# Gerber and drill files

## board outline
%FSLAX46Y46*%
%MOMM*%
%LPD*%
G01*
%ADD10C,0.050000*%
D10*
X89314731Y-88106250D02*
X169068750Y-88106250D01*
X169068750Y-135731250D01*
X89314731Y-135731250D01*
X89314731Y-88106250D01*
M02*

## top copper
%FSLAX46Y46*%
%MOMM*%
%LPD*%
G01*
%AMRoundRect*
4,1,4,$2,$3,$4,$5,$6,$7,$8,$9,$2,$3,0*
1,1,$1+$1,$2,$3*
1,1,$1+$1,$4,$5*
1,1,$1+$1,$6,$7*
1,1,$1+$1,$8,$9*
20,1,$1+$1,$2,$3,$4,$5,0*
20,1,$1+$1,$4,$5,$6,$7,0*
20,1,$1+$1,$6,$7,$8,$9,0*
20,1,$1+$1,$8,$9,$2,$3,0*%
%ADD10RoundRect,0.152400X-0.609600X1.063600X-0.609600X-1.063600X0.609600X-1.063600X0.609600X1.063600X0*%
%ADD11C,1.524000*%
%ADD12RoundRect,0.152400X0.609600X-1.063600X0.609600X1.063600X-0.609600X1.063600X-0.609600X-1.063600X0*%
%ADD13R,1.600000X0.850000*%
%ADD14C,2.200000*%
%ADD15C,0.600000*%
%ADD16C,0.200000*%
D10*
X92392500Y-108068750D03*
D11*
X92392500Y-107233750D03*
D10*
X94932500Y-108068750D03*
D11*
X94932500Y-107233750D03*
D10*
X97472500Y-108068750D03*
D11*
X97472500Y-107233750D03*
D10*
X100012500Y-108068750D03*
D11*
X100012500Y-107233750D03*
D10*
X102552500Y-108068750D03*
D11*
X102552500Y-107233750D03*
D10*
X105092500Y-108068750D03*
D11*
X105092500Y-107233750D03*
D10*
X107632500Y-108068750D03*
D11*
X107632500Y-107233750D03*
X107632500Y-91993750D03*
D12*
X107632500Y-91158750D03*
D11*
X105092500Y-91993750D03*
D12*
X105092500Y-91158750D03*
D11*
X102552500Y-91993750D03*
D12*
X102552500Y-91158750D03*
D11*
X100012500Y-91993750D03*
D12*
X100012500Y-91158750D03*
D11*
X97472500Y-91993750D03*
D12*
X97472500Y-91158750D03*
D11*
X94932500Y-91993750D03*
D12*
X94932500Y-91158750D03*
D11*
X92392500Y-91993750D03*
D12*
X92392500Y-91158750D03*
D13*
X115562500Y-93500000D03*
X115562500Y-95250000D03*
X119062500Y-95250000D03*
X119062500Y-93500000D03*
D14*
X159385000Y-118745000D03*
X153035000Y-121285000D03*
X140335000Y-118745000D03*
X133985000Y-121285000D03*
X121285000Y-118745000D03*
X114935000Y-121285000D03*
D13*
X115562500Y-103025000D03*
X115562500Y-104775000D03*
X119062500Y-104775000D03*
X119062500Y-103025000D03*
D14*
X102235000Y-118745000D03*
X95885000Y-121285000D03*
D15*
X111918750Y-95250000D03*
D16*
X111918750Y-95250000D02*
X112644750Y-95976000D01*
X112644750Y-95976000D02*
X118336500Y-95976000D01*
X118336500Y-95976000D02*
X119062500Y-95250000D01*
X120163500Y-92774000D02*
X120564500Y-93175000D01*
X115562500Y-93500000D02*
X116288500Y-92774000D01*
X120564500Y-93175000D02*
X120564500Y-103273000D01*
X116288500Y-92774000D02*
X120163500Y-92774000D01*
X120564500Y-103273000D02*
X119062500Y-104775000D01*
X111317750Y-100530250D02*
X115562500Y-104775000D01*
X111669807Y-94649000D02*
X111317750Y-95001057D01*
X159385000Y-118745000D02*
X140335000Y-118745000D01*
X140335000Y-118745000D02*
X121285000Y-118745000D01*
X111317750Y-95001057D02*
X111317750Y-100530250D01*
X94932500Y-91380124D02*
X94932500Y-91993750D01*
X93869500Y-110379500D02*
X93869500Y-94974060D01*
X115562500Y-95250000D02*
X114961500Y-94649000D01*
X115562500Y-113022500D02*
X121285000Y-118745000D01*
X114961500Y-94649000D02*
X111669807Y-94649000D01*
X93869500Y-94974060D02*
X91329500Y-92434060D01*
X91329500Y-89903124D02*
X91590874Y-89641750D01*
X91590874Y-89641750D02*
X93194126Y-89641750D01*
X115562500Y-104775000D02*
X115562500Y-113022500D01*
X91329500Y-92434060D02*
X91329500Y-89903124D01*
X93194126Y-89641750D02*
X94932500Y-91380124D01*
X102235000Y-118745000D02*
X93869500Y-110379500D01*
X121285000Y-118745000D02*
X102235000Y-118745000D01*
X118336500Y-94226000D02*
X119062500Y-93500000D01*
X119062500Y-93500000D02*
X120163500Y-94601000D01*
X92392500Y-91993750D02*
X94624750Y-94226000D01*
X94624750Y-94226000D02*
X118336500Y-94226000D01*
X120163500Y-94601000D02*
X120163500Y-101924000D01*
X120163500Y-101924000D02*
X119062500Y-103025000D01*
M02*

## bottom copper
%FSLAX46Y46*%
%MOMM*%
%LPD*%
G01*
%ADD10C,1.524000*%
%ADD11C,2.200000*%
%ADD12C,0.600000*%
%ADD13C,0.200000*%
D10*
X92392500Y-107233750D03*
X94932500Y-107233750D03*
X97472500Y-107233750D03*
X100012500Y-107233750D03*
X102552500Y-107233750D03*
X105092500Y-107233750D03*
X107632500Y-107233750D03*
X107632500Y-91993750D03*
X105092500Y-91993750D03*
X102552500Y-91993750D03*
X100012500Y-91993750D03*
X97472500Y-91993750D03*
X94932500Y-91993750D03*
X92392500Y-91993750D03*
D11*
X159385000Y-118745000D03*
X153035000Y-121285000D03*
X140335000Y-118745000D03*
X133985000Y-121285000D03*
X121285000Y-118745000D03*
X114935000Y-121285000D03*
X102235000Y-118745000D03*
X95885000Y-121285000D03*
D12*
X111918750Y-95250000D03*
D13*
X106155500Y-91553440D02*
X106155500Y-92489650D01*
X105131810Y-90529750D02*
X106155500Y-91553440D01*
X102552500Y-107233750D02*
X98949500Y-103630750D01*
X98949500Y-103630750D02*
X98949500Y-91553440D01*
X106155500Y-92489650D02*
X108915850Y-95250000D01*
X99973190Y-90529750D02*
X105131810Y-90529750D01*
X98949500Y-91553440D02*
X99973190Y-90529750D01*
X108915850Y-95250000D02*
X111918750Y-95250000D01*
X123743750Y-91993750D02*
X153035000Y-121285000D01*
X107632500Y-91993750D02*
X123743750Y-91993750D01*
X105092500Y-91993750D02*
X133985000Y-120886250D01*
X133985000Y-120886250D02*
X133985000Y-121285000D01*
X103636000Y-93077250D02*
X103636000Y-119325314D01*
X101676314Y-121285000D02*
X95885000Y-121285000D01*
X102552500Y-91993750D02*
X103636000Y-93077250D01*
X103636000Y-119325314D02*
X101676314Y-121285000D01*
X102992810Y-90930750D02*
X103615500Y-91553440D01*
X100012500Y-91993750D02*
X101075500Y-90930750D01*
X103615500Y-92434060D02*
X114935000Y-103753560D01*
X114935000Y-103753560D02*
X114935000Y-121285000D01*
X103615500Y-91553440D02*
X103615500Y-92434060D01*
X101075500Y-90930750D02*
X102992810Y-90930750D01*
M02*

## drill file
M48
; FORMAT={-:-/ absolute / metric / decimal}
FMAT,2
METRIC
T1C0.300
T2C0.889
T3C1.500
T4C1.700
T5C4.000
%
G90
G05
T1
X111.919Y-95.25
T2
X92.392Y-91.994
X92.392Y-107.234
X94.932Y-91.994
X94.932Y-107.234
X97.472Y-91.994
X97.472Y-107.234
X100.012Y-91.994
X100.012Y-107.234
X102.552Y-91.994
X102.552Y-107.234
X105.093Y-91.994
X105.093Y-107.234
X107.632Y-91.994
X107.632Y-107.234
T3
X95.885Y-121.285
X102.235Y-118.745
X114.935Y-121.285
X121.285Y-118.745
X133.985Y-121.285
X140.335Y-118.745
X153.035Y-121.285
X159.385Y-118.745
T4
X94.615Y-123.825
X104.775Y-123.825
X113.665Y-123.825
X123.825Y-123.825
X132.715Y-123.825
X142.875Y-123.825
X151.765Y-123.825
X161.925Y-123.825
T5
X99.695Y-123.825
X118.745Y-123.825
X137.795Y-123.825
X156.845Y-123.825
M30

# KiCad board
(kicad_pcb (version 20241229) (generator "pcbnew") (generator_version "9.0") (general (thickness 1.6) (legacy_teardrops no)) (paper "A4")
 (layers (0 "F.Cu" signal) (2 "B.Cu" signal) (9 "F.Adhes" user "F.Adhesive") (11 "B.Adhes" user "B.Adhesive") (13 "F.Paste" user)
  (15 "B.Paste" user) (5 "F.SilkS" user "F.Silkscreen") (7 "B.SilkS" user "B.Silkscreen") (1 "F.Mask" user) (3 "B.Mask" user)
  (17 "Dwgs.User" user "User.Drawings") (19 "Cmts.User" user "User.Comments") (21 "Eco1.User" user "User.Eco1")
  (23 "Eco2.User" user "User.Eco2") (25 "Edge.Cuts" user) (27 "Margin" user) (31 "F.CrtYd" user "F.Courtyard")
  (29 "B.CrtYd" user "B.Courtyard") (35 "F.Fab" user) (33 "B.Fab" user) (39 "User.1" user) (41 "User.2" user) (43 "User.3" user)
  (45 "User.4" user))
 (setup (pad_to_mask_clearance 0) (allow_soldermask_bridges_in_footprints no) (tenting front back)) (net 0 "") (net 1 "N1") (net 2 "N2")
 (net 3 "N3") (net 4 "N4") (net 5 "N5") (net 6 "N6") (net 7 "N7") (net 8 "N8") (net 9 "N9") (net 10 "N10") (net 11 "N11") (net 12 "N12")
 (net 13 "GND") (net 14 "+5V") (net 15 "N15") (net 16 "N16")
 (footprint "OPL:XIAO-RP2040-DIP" (layer "F.Cu") (at 100.0125 99.61375 90)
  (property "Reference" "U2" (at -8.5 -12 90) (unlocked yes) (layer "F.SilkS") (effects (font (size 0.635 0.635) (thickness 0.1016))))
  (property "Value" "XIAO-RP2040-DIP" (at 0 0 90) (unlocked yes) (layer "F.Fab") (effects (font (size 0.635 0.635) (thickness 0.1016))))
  (pad "1" smd roundrect (at -8.455 -7.62 270) (size 2.432 1.524) (layers "F.Cu" "F.Mask") (roundrect_rratio 0.1) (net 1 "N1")
   (thermal_bridge_angle 45))
  (pad "1" thru_hole circle (at -7.62 -7.62 270) (size 1.524 1.524) (drill 0.889) (layers "*.Cu" "*.Mask") (remove_unused_layers no)
   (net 1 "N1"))
  (pad "2" smd roundrect (at -8.455 -5.08 270) (size 2.432 1.524) (layers "F.Cu" "F.Mask") (roundrect_rratio 0.1) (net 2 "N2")
   (thermal_bridge_angle 45))
  (pad "2" thru_hole circle (at -7.62 -5.08 270) (size 1.524 1.524) (drill 0.889) (layers "*.Cu" "*.Mask") (remove_unused_layers no)
   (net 2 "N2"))
  (pad "3" smd roundrect (at -8.455 -2.54 270) (size 2.432 1.524) (layers "F.Cu" "F.Mask") (roundrect_rratio 0.1) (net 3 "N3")
   (thermal_bridge_angle 45))
  (pad "3" thru_hole circle (at -7.62 -2.54 270) (size 1.524 1.524) (drill 0.889) (layers "*.Cu" "*.Mask") (remove_unused_layers no)
   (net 3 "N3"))
  (pad "4" smd roundrect (at -8.455 0 270) (size 2.432 1.524) (layers "F.Cu" "F.Mask") (roundrect_rratio 0.1) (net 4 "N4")
   (thermal_bridge_angle 45))
  (pad "4" thru_hole circle (at -7.62 0 270) (size 1.524 1.524) (drill 0.889) (layers "*.Cu" "*.Mask") (remove_unused_layers no)
   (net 4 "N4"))
  (pad "5" smd roundrect (at -8.455 2.54 270) (size 2.432 1.524) (layers "F.Cu" "F.Mask") (roundrect_rratio 0.1) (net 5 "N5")
   (thermal_bridge_angle 45))
  (pad "5" thru_hole circle (at -7.62 2.54 270) (size 1.524 1.524) (drill 0.889) (layers "*.Cu" "*.Mask") (remove_unused_layers no)
   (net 5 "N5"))
  (pad "6" smd roundrect (at -8.455 5.08 270) (size 2.432 1.524) (layers "F.Cu" "F.Mask") (roundrect_rratio 0.1) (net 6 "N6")
   (thermal_bridge_angle 45))
  (pad "6" thru_hole circle (at -7.62 5.08 270) (size 1.524 1.524) (drill 0.889) (layers "*.Cu" "*.Mask") (remove_unused_layers no)
   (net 6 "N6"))
  (pad "7" smd roundrect (at -8.455 7.62 270) (size 2.432 1.524) (layers "F.Cu" "F.Mask") (roundrect_rratio 0.1) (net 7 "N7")
   (thermal_bridge_angle 45))
  (pad "7" thru_hole circle (at -7.62 7.62 270) (size 1.524 1.524) (drill 0.889) (layers "*.Cu" "*.Mask") (remove_unused_layers no)
   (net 7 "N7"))
  (pad "8" thru_hole circle (at 7.62 7.62 90) (size 1.524 1.524) (drill 0.889) (layers "*.Cu" "*.Mask") (remove_unused_layers no)
   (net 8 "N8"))
  (pad "8" smd roundrect (at 8.455 7.62 90) (size 2.432 1.524) (layers "F.Cu" "F.Mask") (roundrect_rratio 0.1) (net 8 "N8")
   (thermal_bridge_angle 45))
  (pad "9" thru_hole circle (at 7.62 5.08 90) (size 1.524 1.524) (drill 0.889) (layers "*.Cu" "*.Mask") (remove_unused_layers no)
   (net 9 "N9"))
  (pad "9" smd roundrect (at 8.455 5.08 90) (size 2.432 1.524) (layers "F.Cu" "F.Mask") (roundrect_rratio 0.1) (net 9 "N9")
   (thermal_bridge_angle 45))
  (pad "10" thru_hole circle (at 7.62 2.54 90) (size 1.524 1.524) (drill 0.889) (layers "*.Cu" "*.Mask") (remove_unused_layers no)
   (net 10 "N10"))
  (pad "10" smd roundrect (at 8.455 2.54 90) (size 2.432 1.524) (layers "F.Cu" "F.Mask") (roundrect_rratio 0.1) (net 10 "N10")
   (thermal_bridge_angle 45))
  (pad "11" thru_hole circle (at 7.62 0 90) (size 1.524 1.524) (drill 0.889) (layers "*.Cu" "*.Mask") (remove_unused_layers no)
   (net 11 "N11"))
  (pad "11" smd roundrect (at 8.455 0 90) (size 2.432 1.524) (layers "F.Cu" "F.Mask") (roundrect_rratio 0.1) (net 11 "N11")
   (thermal_bridge_angle 45))
  (pad "12" thru_hole circle (at 7.62 -2.54 90) (size 1.524 1.524) (drill 0.889) (layers "*.Cu" "*.Mask") (remove_unused_layers no)
   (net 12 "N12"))
  (pad "12" smd roundrect (at 8.455 -2.54 90) (size 2.432 1.524) (layers "F.Cu" "F.Mask") (roundrect_rratio 0.1) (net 12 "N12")
   (thermal_bridge_angle 45))
  (pad "13" thru_hole circle (at 7.62 -5.08 90) (size 1.524 1.524) (drill 0.889) (layers "*.Cu" "*.Mask") (remove_unused_layers no)
   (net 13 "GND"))
  (pad "13" smd roundrect (at 8.455 -5.08 90) (size 2.432 1.524) (layers "F.Cu" "F.Mask") (roundrect_rratio 0.1) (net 13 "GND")
   (thermal_bridge_angle 45))
  (pad "14" thru_hole circle (at 7.62 -7.62 90) (size 1.524 1.524) (drill 0.889) (layers "*.Cu" "*.Mask") (remove_unused_layers no)
   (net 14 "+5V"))
  (pad "14" smd roundrect (at 8.455 -7.62 90) (size 2.432 1.524) (layers "F.Cu" "F.Mask") (roundrect_rratio 0.1) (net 14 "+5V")
   (thermal_bridge_angle 45)))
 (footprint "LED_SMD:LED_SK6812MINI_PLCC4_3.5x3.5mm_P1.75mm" (layer "F.Cu") (at 117.3125 94.375)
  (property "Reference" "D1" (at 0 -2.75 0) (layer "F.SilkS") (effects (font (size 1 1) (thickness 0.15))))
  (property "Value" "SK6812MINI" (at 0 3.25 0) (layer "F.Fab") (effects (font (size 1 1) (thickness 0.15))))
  (pad "1" smd rect (at -1.75 -0.875) (size 1.6 0.85) (layers "F.Cu" "F.Mask" "F.Paste") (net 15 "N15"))
  (pad "2" smd rect (at -1.75 0.875) (size 1.6 0.85) (layers "F.Cu" "F.Mask" "F.Paste") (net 13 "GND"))
  (pad "3" smd rect (at 1.75 0.875) (size 1.6 0.85) (layers "F.Cu" "F.Mask" "F.Paste") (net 5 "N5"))
  (pad "4" smd rect (at 1.75 -0.875) (size 1.6 0.85) (layers "F.Cu" "F.Mask" "F.Paste") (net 14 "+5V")))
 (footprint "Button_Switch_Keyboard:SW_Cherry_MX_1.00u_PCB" (layer "F.Cu") (at 159.385 118.745)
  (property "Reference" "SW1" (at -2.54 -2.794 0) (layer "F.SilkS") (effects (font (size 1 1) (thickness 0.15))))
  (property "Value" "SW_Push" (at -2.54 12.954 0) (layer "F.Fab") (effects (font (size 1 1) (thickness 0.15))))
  (pad "" np_thru_hole circle (at -7.62 5.08) (size 1.7 1.7) (drill 1.7) (layers "*.Cu" "*.Mask"))
  (pad "" np_thru_hole circle (at -2.54 5.08) (size 4 4) (drill 4) (layers "*.Cu" "*.Mask"))
  (pad "" np_thru_hole circle (at 2.54 5.08) (size 1.7 1.7) (drill 1.7) (layers "*.Cu" "*.Mask"))
  (pad "1" thru_hole circle (at 0 0) (size 2.2 2.2) (drill 1.5) (layers "*.Cu" "*.Mask") (remove_unused_layers no) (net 13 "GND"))
  (pad "2" thru_hole circle (at -6.35 2.54) (size 2.2 2.2) (drill 1.5) (layers "*.Cu" "*.Mask") (remove_unused_layers no) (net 8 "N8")))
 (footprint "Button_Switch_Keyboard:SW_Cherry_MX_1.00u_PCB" (layer "F.Cu") (at 140.335 118.745)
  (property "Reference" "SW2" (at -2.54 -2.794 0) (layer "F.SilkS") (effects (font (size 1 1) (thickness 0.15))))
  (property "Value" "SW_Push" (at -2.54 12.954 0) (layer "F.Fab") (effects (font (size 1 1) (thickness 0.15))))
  (pad "" np_thru_hole circle (at -7.62 5.08) (size 1.7 1.7) (drill 1.7) (layers "*.Cu" "*.Mask"))
  (pad "" np_thru_hole circle (at -2.54 5.08) (size 4 4) (drill 4) (layers "*.Cu" "*.Mask"))
  (pad "" np_thru_hole circle (at 2.54 5.08) (size 1.7 1.7) (drill 1.7) (layers "*.Cu" "*.Mask"))
  (pad "1" thru_hole circle (at 0 0) (size 2.2 2.2) (drill 1.5) (layers "*.Cu" "*.Mask") (remove_unused_layers no) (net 13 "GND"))
  (pad "2" thru_hole circle (at -6.35 2.54) (size 2.2 2.2) (drill 1.5) (layers "*.Cu" "*.Mask") (remove_unused_layers no) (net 9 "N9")))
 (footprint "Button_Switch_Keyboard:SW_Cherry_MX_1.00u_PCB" (layer "F.Cu") (at 121.285 118.745)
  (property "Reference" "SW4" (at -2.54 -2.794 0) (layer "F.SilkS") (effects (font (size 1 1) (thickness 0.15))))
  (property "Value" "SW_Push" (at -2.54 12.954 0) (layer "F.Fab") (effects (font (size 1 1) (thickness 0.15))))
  (pad "" np_thru_hole circle (at -7.62 5.08) (size 1.7 1.7) (drill 1.7) (layers "*.Cu" "*.Mask"))
  (pad "" np_thru_hole circle (at -2.54 5.08) (size 4 4) (drill 4) (layers "*.Cu" "*.Mask"))
  (pad "" np_thru_hole circle (at 2.54 5.08) (size 1.7 1.7) (drill 1.7) (layers "*.Cu" "*.Mask"))
  (pad "1" thru_hole circle (at 0 0) (size 2.2 2.2) (drill 1.5) (layers "*.Cu" "*.Mask") (remove_unused_layers no) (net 13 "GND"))
  (pad "2" thru_hole circle (at -6.35 2.54) (size 2.2 2.2) (drill 1.5) (layers "*.Cu" "*.Mask") (remove_unused_layers no) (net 11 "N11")))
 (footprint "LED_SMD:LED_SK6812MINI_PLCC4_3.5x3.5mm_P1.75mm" (layer "F.Cu") (at 117.3125 103.9)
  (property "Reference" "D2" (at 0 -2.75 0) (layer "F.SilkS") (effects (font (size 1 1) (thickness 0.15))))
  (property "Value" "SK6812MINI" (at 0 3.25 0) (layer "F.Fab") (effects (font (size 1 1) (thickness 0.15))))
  (pad "1" smd rect (at -1.75 -0.875) (size 1.6 0.85) (layers "F.Cu" "F.Mask" "F.Paste") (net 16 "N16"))
  (pad "2" smd rect (at -1.75 0.875) (size 1.6 0.85) (layers "F.Cu" "F.Mask" "F.Paste") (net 13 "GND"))
  (pad "3" smd rect (at 1.75 0.875) (size 1.6 0.85) (layers "F.Cu" "F.Mask" "F.Paste") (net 15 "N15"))
  (pad "4" smd rect (at 1.75 -0.875) (size 1.6 0.85) (layers "F.Cu" "F.Mask" "F.Paste") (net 14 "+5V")))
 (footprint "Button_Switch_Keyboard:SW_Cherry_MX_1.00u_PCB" (layer "F.Cu") (at 102.235 118.745)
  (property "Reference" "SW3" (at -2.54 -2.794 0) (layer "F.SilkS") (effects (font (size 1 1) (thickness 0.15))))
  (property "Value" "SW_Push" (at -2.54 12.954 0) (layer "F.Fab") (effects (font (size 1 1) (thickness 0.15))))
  (pad "" np_thru_hole circle (at -7.62 5.08) (size 1.7 1.7) (drill 1.7) (layers "*.Cu" "*.Mask"))
  (pad "" np_thru_hole circle (at -2.54 5.08) (size 4 4) (drill 4) (layers "*.Cu" "*.Mask"))
  (pad "" np_thru_hole circle (at 2.54 5.08) (size 1.7 1.7) (drill 1.7) (layers "*.Cu" "*.Mask"))
  (pad "1" thru_hole circle (at 0 0) (size 2.2 2.2) (drill 1.5) (layers "*.Cu" "*.Mask") (remove_unused_layers no) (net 13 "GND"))
  (pad "2" thru_hole circle (at -6.35 2.54) (size 2.2 2.2) (drill 1.5) (layers "*.Cu" "*.Mask") (remove_unused_layers no) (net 10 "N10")))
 (gr_rect (start 89.314731 88.10625) (end 169.06875 135.73125) (stroke (width 0.05) (type default)) (fill no) (layer "Edge.Cuts"))
 (segment (start 111.91875 95.25) (end 112.64475 95.976) (width 0.2) (layer "F.Cu") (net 5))
 (segment (start 112.64475 95.976) (end 118.3365 95.976) (width 0.2) (layer "F.Cu") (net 5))
 (segment (start 118.3365 95.976) (end 119.0625 95.25) (width 0.2) (layer "F.Cu") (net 5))
 (via (at 111.91875 95.25) (size 0.6) (drill 0.3) (layers "F.Cu" "B.Cu") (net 5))
 (segment (start 106.1555 91.55344) (end 106.1555 92.48965) (width 0.2) (layer "B.Cu") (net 5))
 (segment (start 105.13181 90.52975) (end 106.1555 91.55344) (width 0.2) (layer "B.Cu") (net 5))
 (segment (start 102.5525 107.23375) (end 98.9495 103.63075) (width 0.2) (layer "B.Cu") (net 5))
 (segment (start 98.9495 103.63075) (end 98.9495 91.55344) (width 0.2) (layer "B.Cu") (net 5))
 (segment (start 106.1555 92.48965) (end 108.91585 95.25) (width 0.2) (layer "B.Cu") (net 5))
 (segment (start 99.97319 90.52975) (end 105.13181 90.52975) (width 0.2) (layer "B.Cu") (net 5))
 (segment (start 98.9495 91.55344) (end 99.97319 90.52975) (width 0.2) (layer "B.Cu") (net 5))
 (segment (start 108.91585 95.25) (end 111.91875 95.25) (width 0.2) (layer "B.Cu") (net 5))
 (segment (start 120.1635 92.774) (end 120.5645 93.175) (width 0.2) (layer "F.Cu") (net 15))
 (segment (start 115.5625 93.5) (end 116.2885 92.774) (width 0.2) (layer "F.Cu") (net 15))
 (segment (start 120.5645 93.175) (end 120.5645 103.273) (width 0.2) (layer "F.Cu") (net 15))
 (segment (start 116.2885 92.774) (end 120.1635 92.774) (width 0.2) (layer "F.Cu") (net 15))
 (segment (start 120.5645 103.273) (end 119.0625 104.775) (width 0.2) (layer "F.Cu") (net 15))
 (segment (start 123.74375 91.99375) (end 153.035 121.285) (width 0.2) (layer "B.Cu") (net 8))
 (segment (start 107.6325 91.99375) (end 123.74375 91.99375) (width 0.2) (layer "B.Cu") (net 8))
 (segment (start 111.31775 100.53025) (end 115.5625 104.775) (width 0.2) (layer "F.Cu") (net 13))
 (segment (start 111.669807 94.649) (end 111.31775 95.001057) (width 0.2) (layer "F.Cu") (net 13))
 (segment (start 159.385 118.745) (end 140.335 118.745) (width 0.2) (layer "F.Cu") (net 13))
 (segment (start 140.335 118.745) (end 121.285 118.745) (width 0.2) (layer "F.Cu") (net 13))
 (segment (start 111.31775 95.001057) (end 111.31775 100.53025) (width 0.2) (layer "F.Cu") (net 13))
 (segment (start 94.9325 91.380124) (end 94.9325 91.99375) (width 0.2) (layer "F.Cu") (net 13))
 (segment (start 93.8695 110.3795) (end 93.8695 94.97406) (width 0.2) (layer "F.Cu") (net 13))
 (segment (start 115.5625 95.25) (end 114.9615 94.649) (width 0.2) (layer "F.Cu") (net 13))
 (segment (start 115.5625 113.0225) (end 121.285 118.745) (width 0.2) (layer "F.Cu") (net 13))
 (segment (start 114.9615 94.649) (end 111.669807 94.649) (width 0.2) (layer "F.Cu") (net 13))
 (segment (start 93.8695 94.97406) (end 91.3295 92.43406) (width 0.2) (layer "F.Cu") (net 13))
 (segment (start 91.3295 89.903124) (end 91.590874 89.64175) (width 0.2) (layer "F.Cu") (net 13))
 (segment (start 91.590874 89.64175) (end 93.194126 89.64175) (width 0.2) (layer "F.Cu") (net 13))
 (segment (start 115.5625 104.775) (end 115.5625 113.0225) (width 0.2) (layer "F.Cu") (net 13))
 (segment (start 91.3295 92.43406) (end 91.3295 89.903124) (width 0.2) (layer "F.Cu") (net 13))
 (segment (start 93.194126 89.64175) (end 94.9325 91.380124) (width 0.2) (layer "F.Cu") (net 13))
 (segment (start 102.235 118.745) (end 93.8695 110.3795) (width 0.2) (layer "F.Cu") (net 13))
 (segment (start 121.285 118.745) (end 102.235 118.745) (width 0.2) (layer "F.Cu") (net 13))
 (segment (start 105.0925 91.99375) (end 133.985 120.88625) (width 0.2) (layer "B.Cu") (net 9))
 (segment (start 133.985 120.88625) (end 133.985 121.285) (width 0.2) (layer "B.Cu") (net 9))
 (segment (start 103.636 93.07725) (end 103.636 119.325314) (width 0.2) (layer "B.Cu") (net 10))
 (segment (start 101.676314 121.285) (end 95.885 121.285) (width 0.2) (layer "B.Cu") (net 10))
 (segment (start 102.5525 91.99375) (end 103.636 93.07725) (width 0.2) (layer "B.Cu") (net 10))
 (segment (start 103.636 119.325314) (end 101.676314 121.285) (width 0.2) (layer "B.Cu") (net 10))
 (segment (start 102.99281 90.93075) (end 103.6155 91.55344) (width 0.2) (layer "B.Cu") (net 11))
 (segment (start 100.0125 91.99375) (end 101.0755 90.93075) (width 0.2) (layer "B.Cu") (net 11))
 (segment (start 103.6155 92.43406) (end 114.935 103.75356) (width 0.2) (layer "B.Cu") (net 11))
 (segment (start 114.935 103.75356) (end 114.935 121.285) (width 0.2) (layer "B.Cu") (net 11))
 (segment (start 103.6155 91.55344) (end 103.6155 92.43406) (width 0.2) (layer "B.Cu") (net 11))
 (segment (start 101.0755 90.93075) (end 102.99281 90.93075) (width 0.2) (layer "B.Cu") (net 11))
 (segment (start 118.3365 94.226) (end 119.0625 93.5) (width 0.2) (layer "F.Cu") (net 14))
 (segment (start 119.0625 93.5) (end 120.1635 94.601) (width 0.2) (layer "F.Cu") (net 14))
 (segment (start 92.3925 91.99375) (end 94.62475 94.226) (width 0.2) (layer "F.Cu") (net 14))
 (segment (start 94.62475 94.226) (end 118.3365 94.226) (width 0.2) (layer "F.Cu") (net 14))
 (segment (start 120.1635 94.601) (end 120.1635 101.924) (width 0.2) (layer "F.Cu") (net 14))
 (segment (start 120.1635 101.924) (end 119.0625 103.025) (width 0.2) (layer "F.Cu") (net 14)))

